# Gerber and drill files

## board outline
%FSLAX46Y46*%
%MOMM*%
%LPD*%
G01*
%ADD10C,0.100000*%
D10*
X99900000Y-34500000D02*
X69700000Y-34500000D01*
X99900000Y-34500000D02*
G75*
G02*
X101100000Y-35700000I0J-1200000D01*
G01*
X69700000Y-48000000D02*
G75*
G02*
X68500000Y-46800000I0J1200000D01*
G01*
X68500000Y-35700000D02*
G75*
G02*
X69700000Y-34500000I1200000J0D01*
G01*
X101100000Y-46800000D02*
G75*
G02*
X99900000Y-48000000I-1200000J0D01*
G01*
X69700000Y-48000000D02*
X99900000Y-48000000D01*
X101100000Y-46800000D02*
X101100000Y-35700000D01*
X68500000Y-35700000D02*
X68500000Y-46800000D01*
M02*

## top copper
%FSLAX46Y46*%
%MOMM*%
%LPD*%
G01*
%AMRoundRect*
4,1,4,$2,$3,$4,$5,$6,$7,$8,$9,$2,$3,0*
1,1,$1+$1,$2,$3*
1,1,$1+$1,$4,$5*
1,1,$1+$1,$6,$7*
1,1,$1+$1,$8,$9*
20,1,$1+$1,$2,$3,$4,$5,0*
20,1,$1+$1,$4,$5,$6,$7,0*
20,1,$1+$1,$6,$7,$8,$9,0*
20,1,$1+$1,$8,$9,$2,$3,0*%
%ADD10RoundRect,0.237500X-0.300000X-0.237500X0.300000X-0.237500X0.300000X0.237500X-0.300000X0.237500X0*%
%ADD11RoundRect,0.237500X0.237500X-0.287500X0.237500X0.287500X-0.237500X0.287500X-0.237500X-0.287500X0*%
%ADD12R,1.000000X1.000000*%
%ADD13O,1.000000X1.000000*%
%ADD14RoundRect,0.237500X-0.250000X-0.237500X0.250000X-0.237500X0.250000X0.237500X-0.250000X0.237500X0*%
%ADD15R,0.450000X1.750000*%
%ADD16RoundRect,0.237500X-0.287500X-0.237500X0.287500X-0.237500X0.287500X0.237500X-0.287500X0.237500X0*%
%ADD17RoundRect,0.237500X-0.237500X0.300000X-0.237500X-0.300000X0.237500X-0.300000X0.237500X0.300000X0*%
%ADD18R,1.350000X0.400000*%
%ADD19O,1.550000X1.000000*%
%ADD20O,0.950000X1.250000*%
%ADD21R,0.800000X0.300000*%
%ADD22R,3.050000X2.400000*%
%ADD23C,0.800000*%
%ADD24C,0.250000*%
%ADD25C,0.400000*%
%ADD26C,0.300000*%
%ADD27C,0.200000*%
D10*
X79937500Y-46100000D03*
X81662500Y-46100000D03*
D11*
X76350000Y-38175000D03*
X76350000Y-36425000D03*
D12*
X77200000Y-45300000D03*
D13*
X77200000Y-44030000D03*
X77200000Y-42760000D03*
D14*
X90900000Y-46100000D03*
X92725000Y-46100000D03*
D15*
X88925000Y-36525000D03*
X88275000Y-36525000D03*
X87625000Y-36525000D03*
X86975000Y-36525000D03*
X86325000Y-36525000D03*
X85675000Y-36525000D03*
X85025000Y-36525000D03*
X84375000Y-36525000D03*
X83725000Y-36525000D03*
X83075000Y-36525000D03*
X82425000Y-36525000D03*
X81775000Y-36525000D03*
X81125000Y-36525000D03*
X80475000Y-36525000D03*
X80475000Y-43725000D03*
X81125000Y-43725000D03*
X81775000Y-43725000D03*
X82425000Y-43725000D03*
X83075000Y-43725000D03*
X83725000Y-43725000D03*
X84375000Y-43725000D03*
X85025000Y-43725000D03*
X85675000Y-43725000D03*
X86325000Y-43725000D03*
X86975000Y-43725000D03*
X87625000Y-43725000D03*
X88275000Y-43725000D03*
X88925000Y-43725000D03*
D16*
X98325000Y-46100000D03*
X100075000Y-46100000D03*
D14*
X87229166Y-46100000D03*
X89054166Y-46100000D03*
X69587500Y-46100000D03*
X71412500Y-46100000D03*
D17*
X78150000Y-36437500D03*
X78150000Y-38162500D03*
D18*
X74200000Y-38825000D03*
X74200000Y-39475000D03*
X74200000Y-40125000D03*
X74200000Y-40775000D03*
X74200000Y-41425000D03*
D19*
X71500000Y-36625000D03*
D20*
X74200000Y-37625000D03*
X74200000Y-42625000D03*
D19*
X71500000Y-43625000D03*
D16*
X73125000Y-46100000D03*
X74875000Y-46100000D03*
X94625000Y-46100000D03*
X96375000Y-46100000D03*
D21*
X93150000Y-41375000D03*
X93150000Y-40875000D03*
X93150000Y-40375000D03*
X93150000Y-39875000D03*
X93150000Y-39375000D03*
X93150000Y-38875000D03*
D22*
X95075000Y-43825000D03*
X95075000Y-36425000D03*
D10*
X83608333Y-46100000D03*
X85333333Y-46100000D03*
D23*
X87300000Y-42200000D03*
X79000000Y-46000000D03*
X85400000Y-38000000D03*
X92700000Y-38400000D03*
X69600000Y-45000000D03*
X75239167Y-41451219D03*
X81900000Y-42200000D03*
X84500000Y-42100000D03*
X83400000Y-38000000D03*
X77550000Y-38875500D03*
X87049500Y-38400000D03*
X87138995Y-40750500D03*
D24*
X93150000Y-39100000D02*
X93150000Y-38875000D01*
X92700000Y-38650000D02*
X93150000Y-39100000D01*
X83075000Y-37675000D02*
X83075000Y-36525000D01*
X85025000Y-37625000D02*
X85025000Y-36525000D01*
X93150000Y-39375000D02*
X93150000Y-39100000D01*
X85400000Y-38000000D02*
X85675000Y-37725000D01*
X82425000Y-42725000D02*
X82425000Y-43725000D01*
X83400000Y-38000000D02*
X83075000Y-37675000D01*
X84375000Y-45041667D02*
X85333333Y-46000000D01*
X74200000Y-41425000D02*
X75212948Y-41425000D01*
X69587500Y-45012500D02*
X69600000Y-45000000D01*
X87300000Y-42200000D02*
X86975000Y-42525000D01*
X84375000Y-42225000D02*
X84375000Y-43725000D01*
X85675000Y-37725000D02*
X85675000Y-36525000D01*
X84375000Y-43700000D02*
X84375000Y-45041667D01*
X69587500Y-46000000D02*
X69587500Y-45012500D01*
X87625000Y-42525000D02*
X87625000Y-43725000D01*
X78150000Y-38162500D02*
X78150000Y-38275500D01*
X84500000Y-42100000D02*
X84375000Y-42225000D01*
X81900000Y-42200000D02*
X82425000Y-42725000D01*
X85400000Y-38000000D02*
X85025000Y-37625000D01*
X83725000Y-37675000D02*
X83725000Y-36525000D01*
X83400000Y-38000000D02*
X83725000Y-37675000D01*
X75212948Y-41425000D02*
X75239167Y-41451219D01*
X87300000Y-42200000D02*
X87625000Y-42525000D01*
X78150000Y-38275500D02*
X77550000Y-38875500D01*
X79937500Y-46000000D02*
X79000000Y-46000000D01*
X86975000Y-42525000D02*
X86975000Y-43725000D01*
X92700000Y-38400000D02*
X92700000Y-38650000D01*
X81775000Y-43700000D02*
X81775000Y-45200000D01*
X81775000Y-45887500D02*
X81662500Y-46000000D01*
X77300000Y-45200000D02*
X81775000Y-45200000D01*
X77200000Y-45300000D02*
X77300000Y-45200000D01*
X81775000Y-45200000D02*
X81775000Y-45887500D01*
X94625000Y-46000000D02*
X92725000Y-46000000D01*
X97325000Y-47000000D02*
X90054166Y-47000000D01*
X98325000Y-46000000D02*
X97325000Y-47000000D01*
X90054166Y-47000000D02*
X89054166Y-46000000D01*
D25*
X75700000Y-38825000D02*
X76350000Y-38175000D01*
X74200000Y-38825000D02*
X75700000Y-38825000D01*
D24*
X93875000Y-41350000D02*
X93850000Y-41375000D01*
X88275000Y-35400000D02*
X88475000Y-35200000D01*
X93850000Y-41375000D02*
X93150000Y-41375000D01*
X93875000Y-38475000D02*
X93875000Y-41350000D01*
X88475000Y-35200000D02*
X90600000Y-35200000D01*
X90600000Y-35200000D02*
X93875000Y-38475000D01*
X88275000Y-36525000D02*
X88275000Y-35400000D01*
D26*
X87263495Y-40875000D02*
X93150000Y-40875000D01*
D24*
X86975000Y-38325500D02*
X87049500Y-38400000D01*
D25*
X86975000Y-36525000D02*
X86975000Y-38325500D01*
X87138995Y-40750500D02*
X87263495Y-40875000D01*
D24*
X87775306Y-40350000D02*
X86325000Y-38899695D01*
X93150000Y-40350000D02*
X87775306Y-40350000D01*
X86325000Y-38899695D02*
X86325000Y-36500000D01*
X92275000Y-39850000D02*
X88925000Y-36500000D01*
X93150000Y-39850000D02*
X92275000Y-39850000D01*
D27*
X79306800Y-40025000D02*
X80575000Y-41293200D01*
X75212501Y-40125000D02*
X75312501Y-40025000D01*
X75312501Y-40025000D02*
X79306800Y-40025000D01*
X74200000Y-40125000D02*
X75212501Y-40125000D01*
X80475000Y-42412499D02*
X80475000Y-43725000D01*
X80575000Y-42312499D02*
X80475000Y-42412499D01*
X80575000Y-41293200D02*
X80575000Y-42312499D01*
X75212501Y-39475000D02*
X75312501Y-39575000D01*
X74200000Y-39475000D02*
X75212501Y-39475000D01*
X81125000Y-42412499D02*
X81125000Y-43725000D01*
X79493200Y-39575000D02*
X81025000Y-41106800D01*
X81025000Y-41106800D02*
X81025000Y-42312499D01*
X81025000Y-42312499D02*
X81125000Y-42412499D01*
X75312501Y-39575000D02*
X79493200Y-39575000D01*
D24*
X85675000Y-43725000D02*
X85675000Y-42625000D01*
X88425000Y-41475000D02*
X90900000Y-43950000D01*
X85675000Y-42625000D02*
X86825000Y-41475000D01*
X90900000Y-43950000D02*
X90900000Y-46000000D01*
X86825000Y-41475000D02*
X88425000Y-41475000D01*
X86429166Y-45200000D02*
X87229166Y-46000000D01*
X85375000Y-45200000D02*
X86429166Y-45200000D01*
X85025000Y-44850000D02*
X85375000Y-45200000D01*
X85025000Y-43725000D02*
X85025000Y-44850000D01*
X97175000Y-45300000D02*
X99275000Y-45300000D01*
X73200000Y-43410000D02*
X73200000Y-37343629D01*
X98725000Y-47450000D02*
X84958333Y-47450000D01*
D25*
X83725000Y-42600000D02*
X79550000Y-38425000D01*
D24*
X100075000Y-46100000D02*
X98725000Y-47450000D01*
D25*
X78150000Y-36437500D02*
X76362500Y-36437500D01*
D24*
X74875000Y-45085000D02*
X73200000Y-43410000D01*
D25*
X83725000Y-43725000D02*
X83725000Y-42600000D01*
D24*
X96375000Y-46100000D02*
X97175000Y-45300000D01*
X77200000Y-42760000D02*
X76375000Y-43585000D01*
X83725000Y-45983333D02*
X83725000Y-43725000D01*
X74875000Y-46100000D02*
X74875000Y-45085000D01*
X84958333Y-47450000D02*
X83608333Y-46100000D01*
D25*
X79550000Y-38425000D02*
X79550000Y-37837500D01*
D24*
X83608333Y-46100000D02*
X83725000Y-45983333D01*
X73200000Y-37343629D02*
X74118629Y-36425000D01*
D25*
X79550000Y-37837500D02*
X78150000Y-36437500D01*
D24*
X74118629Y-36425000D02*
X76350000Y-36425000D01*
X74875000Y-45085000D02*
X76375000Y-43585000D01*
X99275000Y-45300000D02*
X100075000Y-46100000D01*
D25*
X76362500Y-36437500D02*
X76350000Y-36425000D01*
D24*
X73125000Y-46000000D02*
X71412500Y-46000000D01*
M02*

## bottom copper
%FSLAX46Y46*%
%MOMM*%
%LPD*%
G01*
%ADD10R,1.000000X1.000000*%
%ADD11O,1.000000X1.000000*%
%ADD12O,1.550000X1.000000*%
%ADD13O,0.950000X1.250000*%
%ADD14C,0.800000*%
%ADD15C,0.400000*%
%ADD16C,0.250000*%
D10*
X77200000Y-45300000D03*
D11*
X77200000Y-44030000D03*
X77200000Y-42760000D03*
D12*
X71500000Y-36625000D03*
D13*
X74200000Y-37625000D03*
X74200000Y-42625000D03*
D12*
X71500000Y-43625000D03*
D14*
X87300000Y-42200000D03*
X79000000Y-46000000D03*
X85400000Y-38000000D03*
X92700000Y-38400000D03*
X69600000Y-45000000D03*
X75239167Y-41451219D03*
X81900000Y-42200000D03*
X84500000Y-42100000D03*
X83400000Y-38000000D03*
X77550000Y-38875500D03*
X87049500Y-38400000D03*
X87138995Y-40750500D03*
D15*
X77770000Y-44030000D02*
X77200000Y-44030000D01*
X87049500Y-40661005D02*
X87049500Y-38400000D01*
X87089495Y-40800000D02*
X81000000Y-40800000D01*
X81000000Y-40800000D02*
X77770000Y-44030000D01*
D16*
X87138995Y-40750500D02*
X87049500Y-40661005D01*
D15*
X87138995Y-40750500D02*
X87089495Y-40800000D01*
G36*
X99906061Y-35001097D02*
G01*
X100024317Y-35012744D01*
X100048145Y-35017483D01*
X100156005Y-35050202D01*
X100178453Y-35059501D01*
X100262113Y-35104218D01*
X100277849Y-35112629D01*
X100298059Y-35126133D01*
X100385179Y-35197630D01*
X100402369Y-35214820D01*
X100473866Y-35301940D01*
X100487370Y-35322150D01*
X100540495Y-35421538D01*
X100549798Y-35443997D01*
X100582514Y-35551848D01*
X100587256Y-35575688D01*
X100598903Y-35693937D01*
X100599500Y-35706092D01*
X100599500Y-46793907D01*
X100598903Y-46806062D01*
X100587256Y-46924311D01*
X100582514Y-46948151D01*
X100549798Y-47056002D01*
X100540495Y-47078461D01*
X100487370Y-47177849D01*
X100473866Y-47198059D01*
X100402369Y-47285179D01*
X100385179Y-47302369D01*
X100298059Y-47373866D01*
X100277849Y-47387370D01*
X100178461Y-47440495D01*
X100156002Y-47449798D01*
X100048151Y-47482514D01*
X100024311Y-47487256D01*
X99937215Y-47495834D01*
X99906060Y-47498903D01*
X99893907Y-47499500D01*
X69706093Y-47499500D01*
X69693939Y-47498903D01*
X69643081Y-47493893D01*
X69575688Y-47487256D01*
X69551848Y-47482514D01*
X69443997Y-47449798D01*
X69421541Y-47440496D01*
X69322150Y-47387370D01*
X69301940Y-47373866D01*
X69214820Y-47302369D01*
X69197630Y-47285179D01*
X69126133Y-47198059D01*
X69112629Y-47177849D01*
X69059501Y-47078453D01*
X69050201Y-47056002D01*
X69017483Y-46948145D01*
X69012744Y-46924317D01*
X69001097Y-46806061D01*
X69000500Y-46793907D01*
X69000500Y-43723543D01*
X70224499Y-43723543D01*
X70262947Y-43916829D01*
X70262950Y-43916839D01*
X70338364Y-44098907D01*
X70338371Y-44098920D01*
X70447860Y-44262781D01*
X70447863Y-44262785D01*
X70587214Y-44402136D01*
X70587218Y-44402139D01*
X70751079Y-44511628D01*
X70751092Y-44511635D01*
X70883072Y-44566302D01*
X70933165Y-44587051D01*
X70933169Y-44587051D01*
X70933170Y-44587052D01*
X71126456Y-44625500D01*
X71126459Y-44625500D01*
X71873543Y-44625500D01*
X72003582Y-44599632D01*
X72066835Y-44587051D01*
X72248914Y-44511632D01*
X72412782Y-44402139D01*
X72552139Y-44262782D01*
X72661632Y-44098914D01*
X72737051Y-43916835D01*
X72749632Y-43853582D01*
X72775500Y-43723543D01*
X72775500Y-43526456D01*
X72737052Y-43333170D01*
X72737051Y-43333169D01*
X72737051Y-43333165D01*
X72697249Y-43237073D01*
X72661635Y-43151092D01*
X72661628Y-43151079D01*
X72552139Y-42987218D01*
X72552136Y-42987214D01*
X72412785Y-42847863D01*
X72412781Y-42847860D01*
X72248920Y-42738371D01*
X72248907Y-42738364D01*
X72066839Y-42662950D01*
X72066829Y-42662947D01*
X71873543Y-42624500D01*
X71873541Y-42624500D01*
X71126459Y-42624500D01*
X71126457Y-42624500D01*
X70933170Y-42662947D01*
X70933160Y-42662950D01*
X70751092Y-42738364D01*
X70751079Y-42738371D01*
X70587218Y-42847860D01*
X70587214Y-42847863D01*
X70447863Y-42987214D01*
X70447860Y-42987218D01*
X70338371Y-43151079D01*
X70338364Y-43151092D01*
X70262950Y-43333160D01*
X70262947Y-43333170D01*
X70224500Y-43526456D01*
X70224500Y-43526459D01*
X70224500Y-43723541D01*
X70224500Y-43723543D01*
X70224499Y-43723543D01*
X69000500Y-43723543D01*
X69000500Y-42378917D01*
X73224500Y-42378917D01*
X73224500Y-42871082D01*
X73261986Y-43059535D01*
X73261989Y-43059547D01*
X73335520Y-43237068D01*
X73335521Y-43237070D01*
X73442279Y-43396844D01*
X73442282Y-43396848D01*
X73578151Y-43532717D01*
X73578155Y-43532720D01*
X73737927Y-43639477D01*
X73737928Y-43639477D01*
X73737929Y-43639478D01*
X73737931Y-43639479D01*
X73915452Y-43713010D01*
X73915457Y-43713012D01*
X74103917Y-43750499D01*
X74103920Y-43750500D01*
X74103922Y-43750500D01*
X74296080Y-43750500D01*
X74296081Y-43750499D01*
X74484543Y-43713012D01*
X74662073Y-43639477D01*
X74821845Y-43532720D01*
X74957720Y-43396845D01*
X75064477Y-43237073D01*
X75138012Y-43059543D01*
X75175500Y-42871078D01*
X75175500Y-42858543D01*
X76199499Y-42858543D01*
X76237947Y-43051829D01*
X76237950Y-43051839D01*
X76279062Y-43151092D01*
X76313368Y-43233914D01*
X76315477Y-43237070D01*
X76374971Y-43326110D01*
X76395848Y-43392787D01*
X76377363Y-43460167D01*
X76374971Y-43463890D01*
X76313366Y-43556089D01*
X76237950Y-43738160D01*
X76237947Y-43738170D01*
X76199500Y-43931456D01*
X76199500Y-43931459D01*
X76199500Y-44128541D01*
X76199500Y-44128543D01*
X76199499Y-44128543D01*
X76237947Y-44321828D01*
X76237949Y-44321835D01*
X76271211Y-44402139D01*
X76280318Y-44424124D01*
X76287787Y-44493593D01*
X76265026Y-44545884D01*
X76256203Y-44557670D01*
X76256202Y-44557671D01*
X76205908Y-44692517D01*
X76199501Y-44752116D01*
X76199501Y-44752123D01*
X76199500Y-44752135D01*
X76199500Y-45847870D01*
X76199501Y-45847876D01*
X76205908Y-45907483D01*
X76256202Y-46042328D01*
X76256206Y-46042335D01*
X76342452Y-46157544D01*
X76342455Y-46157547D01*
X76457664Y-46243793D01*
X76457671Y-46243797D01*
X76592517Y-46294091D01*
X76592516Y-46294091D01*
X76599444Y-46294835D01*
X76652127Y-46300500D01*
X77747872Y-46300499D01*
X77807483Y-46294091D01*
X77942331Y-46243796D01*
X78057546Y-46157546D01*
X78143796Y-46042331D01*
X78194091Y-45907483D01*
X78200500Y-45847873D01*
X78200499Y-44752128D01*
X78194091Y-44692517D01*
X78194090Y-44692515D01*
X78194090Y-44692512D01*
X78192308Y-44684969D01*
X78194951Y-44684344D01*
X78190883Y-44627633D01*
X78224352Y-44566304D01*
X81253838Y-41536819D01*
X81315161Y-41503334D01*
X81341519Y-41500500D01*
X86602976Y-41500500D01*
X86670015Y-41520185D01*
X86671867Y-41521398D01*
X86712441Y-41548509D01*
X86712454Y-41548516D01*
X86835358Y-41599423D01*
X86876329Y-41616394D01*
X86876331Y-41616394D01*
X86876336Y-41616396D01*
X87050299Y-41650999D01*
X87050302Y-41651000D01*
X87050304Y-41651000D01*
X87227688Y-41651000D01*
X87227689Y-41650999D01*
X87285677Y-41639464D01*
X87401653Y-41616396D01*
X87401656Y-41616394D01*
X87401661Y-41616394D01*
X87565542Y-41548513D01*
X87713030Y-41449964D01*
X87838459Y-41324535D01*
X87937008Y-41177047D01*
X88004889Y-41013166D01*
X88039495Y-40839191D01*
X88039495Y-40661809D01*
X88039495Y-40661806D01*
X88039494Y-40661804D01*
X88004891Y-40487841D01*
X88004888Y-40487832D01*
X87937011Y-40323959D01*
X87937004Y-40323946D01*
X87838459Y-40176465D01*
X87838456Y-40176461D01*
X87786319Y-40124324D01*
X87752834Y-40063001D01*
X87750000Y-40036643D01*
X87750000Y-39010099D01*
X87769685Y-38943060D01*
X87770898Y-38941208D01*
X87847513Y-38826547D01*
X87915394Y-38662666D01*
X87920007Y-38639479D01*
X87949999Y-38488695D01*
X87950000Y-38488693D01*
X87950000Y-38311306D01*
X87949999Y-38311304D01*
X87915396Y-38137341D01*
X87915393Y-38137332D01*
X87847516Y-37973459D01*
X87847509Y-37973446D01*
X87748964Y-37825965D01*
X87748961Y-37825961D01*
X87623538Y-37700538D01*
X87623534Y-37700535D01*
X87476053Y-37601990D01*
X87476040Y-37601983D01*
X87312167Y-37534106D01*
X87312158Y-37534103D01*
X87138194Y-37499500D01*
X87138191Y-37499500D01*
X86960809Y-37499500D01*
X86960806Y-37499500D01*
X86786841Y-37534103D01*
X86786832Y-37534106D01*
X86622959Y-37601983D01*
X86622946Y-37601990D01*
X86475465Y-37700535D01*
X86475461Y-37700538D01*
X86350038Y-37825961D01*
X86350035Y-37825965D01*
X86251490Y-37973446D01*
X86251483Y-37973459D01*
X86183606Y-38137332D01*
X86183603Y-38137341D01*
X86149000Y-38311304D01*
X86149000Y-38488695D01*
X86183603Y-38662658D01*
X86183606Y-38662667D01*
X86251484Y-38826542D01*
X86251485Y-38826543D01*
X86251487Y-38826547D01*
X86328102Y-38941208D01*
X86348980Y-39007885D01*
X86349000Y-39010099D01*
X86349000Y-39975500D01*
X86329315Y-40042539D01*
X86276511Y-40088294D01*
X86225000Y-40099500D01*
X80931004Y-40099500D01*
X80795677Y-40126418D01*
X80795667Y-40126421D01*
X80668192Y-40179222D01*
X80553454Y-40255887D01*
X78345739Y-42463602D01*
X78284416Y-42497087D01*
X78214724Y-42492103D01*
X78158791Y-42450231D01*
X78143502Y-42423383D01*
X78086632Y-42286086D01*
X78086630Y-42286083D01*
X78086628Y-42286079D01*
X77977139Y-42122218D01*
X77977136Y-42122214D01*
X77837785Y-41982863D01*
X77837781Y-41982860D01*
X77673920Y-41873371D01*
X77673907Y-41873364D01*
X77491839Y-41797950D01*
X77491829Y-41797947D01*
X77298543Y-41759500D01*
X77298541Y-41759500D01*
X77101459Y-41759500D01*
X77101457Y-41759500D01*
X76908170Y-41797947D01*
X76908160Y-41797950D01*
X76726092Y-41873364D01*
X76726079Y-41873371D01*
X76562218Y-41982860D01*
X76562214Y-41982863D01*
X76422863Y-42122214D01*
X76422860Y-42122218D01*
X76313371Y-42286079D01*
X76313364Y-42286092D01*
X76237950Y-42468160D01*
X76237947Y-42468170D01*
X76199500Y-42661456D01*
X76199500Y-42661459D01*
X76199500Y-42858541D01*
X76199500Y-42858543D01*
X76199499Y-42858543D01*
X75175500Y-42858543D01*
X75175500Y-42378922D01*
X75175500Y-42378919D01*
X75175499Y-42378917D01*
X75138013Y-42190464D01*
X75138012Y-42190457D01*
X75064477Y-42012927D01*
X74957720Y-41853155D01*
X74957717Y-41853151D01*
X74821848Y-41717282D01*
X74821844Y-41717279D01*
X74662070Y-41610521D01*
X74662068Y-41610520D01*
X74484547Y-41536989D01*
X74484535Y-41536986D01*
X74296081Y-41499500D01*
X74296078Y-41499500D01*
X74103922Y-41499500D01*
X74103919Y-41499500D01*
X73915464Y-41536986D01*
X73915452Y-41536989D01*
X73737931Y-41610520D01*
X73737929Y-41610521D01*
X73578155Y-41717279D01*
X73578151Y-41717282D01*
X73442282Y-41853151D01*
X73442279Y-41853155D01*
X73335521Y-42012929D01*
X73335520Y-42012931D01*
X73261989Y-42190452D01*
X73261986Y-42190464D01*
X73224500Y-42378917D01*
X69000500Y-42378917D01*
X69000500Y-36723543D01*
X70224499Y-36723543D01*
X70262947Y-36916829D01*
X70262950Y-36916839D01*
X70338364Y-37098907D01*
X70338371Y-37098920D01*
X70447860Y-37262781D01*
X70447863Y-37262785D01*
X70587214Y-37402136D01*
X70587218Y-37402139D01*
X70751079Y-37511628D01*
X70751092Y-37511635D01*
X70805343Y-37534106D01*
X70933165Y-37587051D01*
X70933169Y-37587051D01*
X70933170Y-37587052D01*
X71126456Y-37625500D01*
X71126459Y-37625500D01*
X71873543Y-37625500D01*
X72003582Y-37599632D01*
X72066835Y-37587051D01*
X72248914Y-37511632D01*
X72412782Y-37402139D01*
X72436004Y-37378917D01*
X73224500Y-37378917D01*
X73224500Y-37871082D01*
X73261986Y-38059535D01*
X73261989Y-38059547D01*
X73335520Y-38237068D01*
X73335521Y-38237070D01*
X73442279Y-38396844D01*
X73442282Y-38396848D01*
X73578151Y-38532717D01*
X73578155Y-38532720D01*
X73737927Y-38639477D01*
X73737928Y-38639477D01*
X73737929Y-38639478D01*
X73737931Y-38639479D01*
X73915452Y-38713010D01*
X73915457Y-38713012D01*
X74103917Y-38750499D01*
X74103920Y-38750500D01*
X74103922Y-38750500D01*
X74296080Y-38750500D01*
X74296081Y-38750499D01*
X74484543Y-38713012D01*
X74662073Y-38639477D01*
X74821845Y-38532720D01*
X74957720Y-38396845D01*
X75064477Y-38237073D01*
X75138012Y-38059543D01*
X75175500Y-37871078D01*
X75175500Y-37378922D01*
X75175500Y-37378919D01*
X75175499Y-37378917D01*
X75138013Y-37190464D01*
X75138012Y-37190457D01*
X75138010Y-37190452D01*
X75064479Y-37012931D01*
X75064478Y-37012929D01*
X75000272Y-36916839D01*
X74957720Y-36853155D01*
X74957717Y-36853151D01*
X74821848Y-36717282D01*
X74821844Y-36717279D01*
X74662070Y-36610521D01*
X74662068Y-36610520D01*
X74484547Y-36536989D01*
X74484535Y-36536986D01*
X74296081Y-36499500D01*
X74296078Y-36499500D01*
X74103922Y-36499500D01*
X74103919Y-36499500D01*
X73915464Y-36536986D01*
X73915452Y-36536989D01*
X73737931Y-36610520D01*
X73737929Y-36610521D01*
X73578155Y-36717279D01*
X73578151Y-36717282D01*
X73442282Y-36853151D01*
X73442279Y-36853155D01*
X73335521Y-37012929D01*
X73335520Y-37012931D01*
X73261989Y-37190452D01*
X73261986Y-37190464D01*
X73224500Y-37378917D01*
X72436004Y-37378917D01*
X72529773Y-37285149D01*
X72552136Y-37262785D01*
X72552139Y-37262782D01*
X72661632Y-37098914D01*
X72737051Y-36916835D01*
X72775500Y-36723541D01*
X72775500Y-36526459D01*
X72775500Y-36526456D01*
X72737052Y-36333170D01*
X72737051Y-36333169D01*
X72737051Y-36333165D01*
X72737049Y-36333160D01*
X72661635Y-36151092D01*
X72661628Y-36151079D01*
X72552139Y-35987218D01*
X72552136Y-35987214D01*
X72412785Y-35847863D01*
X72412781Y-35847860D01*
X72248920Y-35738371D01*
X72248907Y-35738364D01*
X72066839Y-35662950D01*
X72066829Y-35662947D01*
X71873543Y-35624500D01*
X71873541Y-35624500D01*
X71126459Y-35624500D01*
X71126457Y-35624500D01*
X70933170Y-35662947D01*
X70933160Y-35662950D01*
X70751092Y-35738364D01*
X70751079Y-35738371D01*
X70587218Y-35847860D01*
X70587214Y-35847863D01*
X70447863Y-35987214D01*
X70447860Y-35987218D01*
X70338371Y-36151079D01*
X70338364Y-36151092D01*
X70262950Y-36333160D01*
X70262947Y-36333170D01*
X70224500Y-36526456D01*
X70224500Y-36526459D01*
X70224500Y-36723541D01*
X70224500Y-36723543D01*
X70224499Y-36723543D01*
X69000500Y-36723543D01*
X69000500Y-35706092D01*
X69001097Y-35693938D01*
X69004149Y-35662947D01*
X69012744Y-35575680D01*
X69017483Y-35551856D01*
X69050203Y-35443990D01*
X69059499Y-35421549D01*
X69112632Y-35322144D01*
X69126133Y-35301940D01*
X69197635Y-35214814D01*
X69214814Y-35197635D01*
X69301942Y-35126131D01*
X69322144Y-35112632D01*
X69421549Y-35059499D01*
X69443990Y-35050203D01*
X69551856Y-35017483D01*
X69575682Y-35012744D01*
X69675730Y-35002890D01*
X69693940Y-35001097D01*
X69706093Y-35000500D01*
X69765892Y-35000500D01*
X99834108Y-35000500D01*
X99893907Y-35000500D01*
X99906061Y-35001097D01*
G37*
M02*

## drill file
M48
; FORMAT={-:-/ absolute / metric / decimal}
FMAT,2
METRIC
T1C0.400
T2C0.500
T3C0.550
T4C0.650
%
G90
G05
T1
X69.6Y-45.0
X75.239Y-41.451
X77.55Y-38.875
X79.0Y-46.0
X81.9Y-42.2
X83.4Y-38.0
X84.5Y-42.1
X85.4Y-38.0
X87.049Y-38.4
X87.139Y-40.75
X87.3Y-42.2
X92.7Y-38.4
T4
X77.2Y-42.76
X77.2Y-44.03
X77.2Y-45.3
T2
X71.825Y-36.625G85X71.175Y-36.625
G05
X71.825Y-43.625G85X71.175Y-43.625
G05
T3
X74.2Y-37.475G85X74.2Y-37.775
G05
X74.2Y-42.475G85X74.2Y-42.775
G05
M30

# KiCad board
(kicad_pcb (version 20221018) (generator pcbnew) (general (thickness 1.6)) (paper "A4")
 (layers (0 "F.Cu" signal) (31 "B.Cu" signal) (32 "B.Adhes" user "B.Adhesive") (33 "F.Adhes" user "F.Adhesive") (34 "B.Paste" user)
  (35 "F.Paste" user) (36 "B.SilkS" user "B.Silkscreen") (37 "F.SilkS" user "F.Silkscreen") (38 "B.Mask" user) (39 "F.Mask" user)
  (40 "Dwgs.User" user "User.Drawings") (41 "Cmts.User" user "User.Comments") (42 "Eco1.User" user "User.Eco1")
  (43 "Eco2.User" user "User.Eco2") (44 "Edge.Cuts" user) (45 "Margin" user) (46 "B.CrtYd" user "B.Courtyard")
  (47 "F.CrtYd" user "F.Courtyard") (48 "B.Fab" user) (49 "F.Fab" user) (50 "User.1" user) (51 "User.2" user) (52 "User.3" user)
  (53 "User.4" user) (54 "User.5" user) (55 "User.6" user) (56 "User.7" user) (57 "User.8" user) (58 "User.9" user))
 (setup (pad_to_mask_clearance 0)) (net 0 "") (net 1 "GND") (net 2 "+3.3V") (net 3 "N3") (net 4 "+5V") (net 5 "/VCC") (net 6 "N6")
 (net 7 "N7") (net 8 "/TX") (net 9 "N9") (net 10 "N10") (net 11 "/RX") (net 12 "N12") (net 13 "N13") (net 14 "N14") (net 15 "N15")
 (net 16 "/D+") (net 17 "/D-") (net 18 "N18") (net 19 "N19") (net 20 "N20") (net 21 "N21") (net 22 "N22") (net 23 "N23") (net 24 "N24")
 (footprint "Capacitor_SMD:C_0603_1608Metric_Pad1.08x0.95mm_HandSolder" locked (layer "F.Cu") (at 80.8 46.1)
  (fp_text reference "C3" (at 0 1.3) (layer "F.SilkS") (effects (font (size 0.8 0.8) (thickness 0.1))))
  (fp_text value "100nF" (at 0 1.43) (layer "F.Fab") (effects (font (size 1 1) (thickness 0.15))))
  (pad "1" smd roundrect locked (at -0.8625 0) (size 1.075 0.95) (layers "F.Cu" "F.Paste" "F.Mask") (roundrect_rratio 0.25) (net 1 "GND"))
  (pad "2" smd roundrect locked (at 0.8625 0) (size 1.075 0.95) (layers "F.Cu" "F.Paste" "F.Mask") (roundrect_rratio 0.25) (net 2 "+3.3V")))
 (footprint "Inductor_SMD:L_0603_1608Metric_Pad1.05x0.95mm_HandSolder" (layer "F.Cu") (at 76.35 37.3 90)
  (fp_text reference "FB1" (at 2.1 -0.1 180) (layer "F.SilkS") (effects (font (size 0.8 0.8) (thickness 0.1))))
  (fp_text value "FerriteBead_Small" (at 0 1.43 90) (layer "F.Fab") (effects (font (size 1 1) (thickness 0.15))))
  (pad "1" smd roundrect (at -0.875 0 90) (size 1.05 0.95) (layers "F.Cu" "F.Paste" "F.Mask") (roundrect_rratio 0.25) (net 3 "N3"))
  (pad "2" smd roundrect (at 0.875 0 90) (size 1.05 0.95) (layers "F.Cu" "F.Paste" "F.Mask") (roundrect_rratio 0.25) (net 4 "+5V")))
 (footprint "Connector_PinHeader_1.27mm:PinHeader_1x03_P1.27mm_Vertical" (layer "F.Cu") (at 77.2 45.3 180)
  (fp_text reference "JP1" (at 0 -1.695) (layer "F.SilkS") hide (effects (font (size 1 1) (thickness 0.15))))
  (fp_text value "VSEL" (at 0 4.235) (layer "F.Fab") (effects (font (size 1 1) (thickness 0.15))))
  (pad "1" thru_hole rect (at 0 0 180) (size 1 1) (drill 0.65) (layers "*.Cu" "*.Mask") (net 2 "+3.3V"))
  (pad "2" thru_hole oval (at 0 1.27 180) (size 1 1) (drill 0.65) (layers "*.Cu" "*.Mask") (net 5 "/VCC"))
  (pad "3" thru_hole oval (at 0 2.54 180) (size 1 1) (drill 0.65) (layers "*.Cu" "*.Mask") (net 4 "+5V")))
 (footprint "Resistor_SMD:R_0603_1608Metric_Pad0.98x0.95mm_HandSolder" (layer "F.Cu") (at 91.8125 46.1)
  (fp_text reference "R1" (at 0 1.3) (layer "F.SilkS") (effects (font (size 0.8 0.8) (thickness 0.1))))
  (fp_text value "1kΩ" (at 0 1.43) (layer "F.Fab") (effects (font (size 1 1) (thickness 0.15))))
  (pad "1" smd roundrect (at -0.9125 0) (size 0.975 0.95) (layers "F.Cu" "F.Paste" "F.Mask") (roundrect_rratio 0.25) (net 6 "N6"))
  (pad "2" smd roundrect (at 0.9125 0) (size 0.975 0.95) (layers "F.Cu" "F.Paste" "F.Mask") (roundrect_rratio 0.25) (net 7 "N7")))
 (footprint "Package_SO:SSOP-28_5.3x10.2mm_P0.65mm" (layer "F.Cu") (at 84.7 40.125 -90)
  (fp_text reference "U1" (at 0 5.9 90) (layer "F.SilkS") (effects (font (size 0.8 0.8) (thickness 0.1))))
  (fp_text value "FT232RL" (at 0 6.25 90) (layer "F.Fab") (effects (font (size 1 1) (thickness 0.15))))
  (pad "1" smd rect (at -3.6 -4.225 270) (size 1.75 0.45) (layers "F.Cu" "F.Paste" "F.Mask") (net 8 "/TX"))
  (pad "2" smd rect (at -3.6 -3.575 270) (size 1.75 0.45) (layers "F.Cu" "F.Paste" "F.Mask") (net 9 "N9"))
  (pad "3" smd rect (at -3.6 -2.925 270) (size 1.75 0.45) (layers "F.Cu" "F.Paste" "F.Mask") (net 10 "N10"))
  (pad "4" smd rect (at -3.6 -2.275 270) (size 1.75 0.45) (layers "F.Cu" "F.Paste" "F.Mask") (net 5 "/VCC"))
  (pad "5" smd rect (at -3.6 -1.625 270) (size 1.75 0.45) (layers "F.Cu" "F.Paste" "F.Mask") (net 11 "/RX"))
  (pad "6" smd rect (at -3.6 -0.975 270) (size 1.75 0.45) (layers "F.Cu" "F.Paste" "F.Mask") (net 1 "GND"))
  (pad "7" smd rect (at -3.6 -0.325 270) (size 1.75 0.45) (layers "F.Cu" "F.Paste" "F.Mask") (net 1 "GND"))
  (pad "8" smd rect (at -3.6 0.325 270) (size 1.75 0.45) (layers "F.Cu" "F.Paste" "F.Mask"))
  (pad "9" smd rect (at -3.6 0.975 270) (size 1.75 0.45) (layers "F.Cu" "F.Paste" "F.Mask") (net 1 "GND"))
  (pad "10" smd rect (at -3.6 1.625 270) (size 1.75 0.45) (layers "F.Cu" "F.Paste" "F.Mask") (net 1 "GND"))
  (pad "11" smd rect (at -3.6 2.275 270) (size 1.75 0.45) (layers "F.Cu" "F.Paste" "F.Mask") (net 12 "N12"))
  (pad "12" smd rect (at -3.6 2.925 270) (size 1.75 0.45) (layers "F.Cu" "F.Paste" "F.Mask") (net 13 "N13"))
  (pad "13" smd rect (at -3.6 3.575 270) (size 1.75 0.45) (layers "F.Cu" "F.Paste" "F.Mask") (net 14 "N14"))
  (pad "14" smd rect (at -3.6 4.225 270) (size 1.75 0.45) (layers "F.Cu" "F.Paste" "F.Mask") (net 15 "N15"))
  (pad "15" smd rect (at 3.6 4.225 270) (size 1.75 0.45) (layers "F.Cu" "F.Paste" "F.Mask") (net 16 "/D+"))
  (pad "16" smd rect (at 3.6 3.575 270) (size 1.75 0.45) (layers "F.Cu" "F.Paste" "F.Mask") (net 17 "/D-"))
  (pad "17" smd rect (at 3.6 2.925 270) (size 1.75 0.45) (layers "F.Cu" "F.Paste" "F.Mask") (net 2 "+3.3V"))
  (pad "18" smd rect (at 3.6 2.275 270) (size 1.75 0.45) (layers "F.Cu" "F.Paste" "F.Mask") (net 1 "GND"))
  (pad "19" smd rect (at 3.6 1.625 270) (size 1.75 0.45) (layers "F.Cu" "F.Paste" "F.Mask") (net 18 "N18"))
  (pad "20" smd rect (at 3.6 0.975 270) (size 1.75 0.45) (layers "F.Cu" "F.Paste" "F.Mask") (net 4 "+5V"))
  (pad "21" smd rect (at 3.6 0.325 270) (size 1.75 0.45) (layers "F.Cu" "F.Paste" "F.Mask") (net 1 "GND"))
  (pad "22" smd rect (at 3.6 -0.325 270) (size 1.75 0.45) (layers "F.Cu" "F.Paste" "F.Mask") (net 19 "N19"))
  (pad "23" smd rect (at 3.6 -0.975 270) (size 1.75 0.45) (layers "F.Cu" "F.Paste" "F.Mask") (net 6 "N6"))
  (pad "24" smd rect (at 3.6 -1.625 270) (size 1.75 0.45) (layers "F.Cu" "F.Paste" "F.Mask"))
  (pad "25" smd rect (at 3.6 -2.275 270) (size 1.75 0.45) (layers "F.Cu" "F.Paste" "F.Mask") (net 1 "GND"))
  (pad "26" smd rect (at 3.6 -2.925 270) (size 1.75 0.45) (layers "F.Cu" "F.Paste" "F.Mask") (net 1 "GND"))
  (pad "27" smd rect (at 3.6 -3.575 270) (size 1.75 0.45) (layers "F.Cu" "F.Paste" "F.Mask") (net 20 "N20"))
  (pad "28" smd rect (at 3.6 -4.225 270) (size 1.75 0.45) (layers "F.Cu" "F.Paste" "F.Mask") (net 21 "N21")))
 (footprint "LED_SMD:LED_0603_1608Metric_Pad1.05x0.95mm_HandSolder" (layer "F.Cu") (at 99.2 46.1)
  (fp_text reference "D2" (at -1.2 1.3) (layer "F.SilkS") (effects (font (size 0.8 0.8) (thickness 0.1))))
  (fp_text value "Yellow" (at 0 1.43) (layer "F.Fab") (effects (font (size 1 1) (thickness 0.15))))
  (pad "1" smd roundrect (at -0.875 0) (size 1.05 0.95) (layers "F.Cu" "F.Paste" "F.Mask") (roundrect_rratio 0.25) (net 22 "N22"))
  (pad "2" smd roundrect (at 0.875 0) (size 1.05 0.95) (layers "F.Cu" "F.Paste" "F.Mask") (roundrect_rratio 0.25) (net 4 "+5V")))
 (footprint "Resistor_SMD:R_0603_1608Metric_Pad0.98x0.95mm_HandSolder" (layer "F.Cu") (at 88.141666 46.1)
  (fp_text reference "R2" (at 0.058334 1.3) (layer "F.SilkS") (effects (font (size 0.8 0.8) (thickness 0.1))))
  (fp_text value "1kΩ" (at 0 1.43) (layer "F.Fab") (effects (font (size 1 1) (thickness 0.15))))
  (pad "1" smd roundrect (at -0.9125 0) (size 0.975 0.95) (layers "F.Cu" "F.Paste" "F.Mask") (roundrect_rratio 0.25) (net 19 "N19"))
  (pad "2" smd roundrect (at 0.9125 0) (size 0.975 0.95) (layers "F.Cu" "F.Paste" "F.Mask") (roundrect_rratio 0.25) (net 22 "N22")))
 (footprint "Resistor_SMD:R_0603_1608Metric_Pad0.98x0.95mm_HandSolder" (layer "F.Cu") (at 70.5 46.1)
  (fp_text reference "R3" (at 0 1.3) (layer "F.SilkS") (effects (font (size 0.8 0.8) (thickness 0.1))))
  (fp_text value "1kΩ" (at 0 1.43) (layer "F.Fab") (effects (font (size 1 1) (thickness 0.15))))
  (pad "1" smd roundrect (at -0.9125 0) (size 0.975 0.95) (layers "F.Cu" "F.Paste" "F.Mask") (roundrect_rratio 0.25) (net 1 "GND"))
  (pad "2" smd roundrect (at 0.9125 0) (size 0.975 0.95) (layers "F.Cu" "F.Paste" "F.Mask") (roundrect_rratio 0.25) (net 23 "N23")))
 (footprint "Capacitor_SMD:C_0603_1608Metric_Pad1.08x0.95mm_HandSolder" (layer "F.Cu") (at 78.15 37.3 -90)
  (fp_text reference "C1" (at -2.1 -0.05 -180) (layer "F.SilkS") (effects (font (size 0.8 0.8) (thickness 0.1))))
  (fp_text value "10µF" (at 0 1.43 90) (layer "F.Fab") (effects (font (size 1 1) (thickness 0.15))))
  (pad "1" smd roundrect (at -0.8625 0 270) (size 1.075 0.95) (layers "F.Cu" "F.Paste" "F.Mask") (roundrect_rratio 0.25) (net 4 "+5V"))
  (pad "2" smd roundrect (at 0.8625 0 270) (size 1.075 0.95) (layers "F.Cu" "F.Paste" "F.Mask") (roundrect_rratio 0.25) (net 1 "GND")))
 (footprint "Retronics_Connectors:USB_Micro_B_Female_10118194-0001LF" (layer "F.Cu") (at 74.2 40.125 -90)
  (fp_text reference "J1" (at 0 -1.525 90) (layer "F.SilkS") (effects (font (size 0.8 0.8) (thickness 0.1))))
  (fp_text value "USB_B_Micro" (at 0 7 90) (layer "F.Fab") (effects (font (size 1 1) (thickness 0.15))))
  (pad "1" smd rect (at -1.3 0 270) (size 0.4 1.35) (layers "F.Cu" "F.Paste" "F.Mask") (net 3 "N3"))
  (pad "2" smd rect (at -0.65 0 270) (size 0.4 1.35) (layers "F.Cu" "F.Paste" "F.Mask") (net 17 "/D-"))
  (pad "3" smd rect (at 0 0 270) (size 0.4 1.35) (layers "F.Cu" "F.Paste" "F.Mask") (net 16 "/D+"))
  (pad "4" smd rect (at 0.65 0 270) (size 0.4 1.35) (layers "F.Cu" "F.Paste" "F.Mask") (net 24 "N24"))
  (pad "5" smd rect (at 1.3 0 270) (size 0.4 1.35) (layers "F.Cu" "F.Paste" "F.Mask") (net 1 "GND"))
  (pad "SH" thru_hole oval (at -3.5 2.7 270) (size 1 1.55) (drill oval 0.5 1.15) (layers "*.Cu" "*.Mask"))
  (pad "SH" thru_hole oval (at -2.5 0 270) (size 1.25 0.95) (drill oval 0.85 0.55) (layers "*.Cu" "*.Mask"))
  (pad "SH" thru_hole oval (at 2.5 0 270) (size 1.25 0.95) (drill oval 0.85 0.55) (layers "*.Cu" "*.Mask"))
  (pad "SH" thru_hole oval (at 3.5 2.7 270) (size 1 1.55) (drill oval 0.5 1.15) (layers "*.Cu" "*.Mask")))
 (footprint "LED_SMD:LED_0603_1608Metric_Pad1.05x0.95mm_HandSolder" (layer "F.Cu") (at 74 46.1)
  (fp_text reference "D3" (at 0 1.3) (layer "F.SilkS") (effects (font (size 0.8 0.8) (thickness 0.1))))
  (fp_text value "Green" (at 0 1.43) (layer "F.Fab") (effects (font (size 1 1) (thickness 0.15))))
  (pad "1" smd roundrect (at -0.875 0) (size 1.05 0.95) (layers "F.Cu" "F.Paste" "F.Mask") (roundrect_rratio 0.25) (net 23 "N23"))
  (pad "2" smd roundrect (at 0.875 0) (size 1.05 0.95) (layers "F.Cu" "F.Paste" "F.Mask") (roundrect_rratio 0.25) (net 4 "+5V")))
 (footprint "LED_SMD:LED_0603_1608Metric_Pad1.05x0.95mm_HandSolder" (layer "F.Cu") (at 95.5 46.1)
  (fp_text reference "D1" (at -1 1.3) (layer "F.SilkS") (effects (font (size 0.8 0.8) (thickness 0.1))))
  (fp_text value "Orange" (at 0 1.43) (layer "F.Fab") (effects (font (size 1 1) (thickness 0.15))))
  (pad "1" smd roundrect (at -0.875 0) (size 1.05 0.95) (layers "F.Cu" "F.Paste" "F.Mask") (roundrect_rratio 0.25) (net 7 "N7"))
  (pad "2" smd roundrect (at 0.875 0) (size 1.05 0.95) (layers "F.Cu" "F.Paste" "F.Mask") (roundrect_rratio 0.25) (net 4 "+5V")))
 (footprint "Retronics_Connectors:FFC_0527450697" (layer "F.Cu") (at 96.1 40.125 90)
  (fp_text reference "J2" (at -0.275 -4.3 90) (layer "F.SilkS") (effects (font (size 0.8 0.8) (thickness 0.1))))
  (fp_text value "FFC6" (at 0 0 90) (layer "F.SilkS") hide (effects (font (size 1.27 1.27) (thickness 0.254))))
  (pad "1" smd rect (at -1.25 -2.95 90) (size 0.3 0.8) (layers "F.Cu" "F.Paste" "F.Mask") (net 9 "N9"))
  (pad "2" smd rect (at -0.75 -2.95 90) (size 0.3 0.8) (layers "F.Cu" "F.Paste" "F.Mask") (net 5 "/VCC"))
  (pad "3" smd rect (at -0.25 -2.95 90) (size 0.3 0.8) (layers "F.Cu" "F.Paste" "F.Mask") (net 11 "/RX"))
  (pad "4" smd rect (at 0.25 -2.95 90) (size 0.3 0.8) (layers "F.Cu" "F.Paste" "F.Mask") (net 8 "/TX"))
  (pad "5" smd rect (at 0.75 -2.95 90) (size 0.3 0.8) (layers "F.Cu" "F.Paste" "F.Mask") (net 1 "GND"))
  (pad "6" smd rect (at 1.25 -2.95 90) (size 0.3 0.8) (layers "F.Cu" "F.Paste" "F.Mask") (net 1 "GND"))
  (pad "7" smd rect (at -3.7 -1.025 90) (size 2.4 3.05) (layers "F.Cu" "F.Paste" "F.Mask"))
  (pad "8" smd rect (at 3.7 -1.025 90) (size 2.4 3.05) (layers "F.Cu" "F.Paste" "F.Mask")))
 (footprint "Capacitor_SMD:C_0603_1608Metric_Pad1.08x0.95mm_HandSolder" (layer "F.Cu") (at 84.470833 46.1)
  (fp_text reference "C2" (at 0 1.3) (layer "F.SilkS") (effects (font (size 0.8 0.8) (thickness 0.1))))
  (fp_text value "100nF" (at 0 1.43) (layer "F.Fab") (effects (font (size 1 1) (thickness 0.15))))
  (pad "1" smd roundrect (at -0.8625 0) (size 1.075 0.95) (layers "F.Cu" "F.Paste" "F.Mask") (roundrect_rratio 0.25) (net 4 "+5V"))
  (pad "2" smd roundrect (at 0.8625 0) (size 1.075 0.95) (layers "F.Cu" "F.Paste" "F.Mask") (roundrect_rratio 0.25) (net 1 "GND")))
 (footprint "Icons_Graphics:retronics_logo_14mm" (layer "B.Cu") (at 93.996672 35.9 180)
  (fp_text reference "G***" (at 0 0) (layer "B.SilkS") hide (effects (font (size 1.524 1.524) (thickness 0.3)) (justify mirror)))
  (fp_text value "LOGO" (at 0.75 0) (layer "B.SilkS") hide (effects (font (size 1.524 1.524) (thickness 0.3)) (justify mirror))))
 (gr_line (start 99.9 34.5) (end 69.7 34.5) (stroke (width 0.1) (type default)) (layer "Edge.Cuts"))
 (gr_arc (start 99.9 34.5) (mid 100.748528 34.851472) (end 101.1 35.7) (stroke (width 0.1) (type default)) (layer "Edge.Cuts"))
 (gr_arc (start 69.7 48) (mid 68.851472 47.648528) (end 68.5 46.8) (stroke (width 0.1) (type default)) (layer "Edge.Cuts"))
 (gr_arc (start 68.5 35.7) (mid 68.851472 34.851472) (end 69.7 34.5) (stroke (width 0.1) (type default)) (layer "Edge.Cuts"))
 (gr_arc (start 101.1 46.8) (mid 100.748528 47.648528) (end 99.9 48) (stroke (width 0.1) (type default)) (layer "Edge.Cuts"))
 (gr_line (start 69.7 48) (end 99.9 48) (stroke (width 0.1) (type default)) (layer "Edge.Cuts"))
 (gr_line (start 101.1 46.8) (end 101.1 35.7) (stroke (width 0.1) (type default)) (layer "Edge.Cuts"))
 (gr_line (start 68.5 35.7) (end 68.5 46.8) (stroke (width 0.1) (type default)) (layer "Edge.Cuts"))
 (segment (start 93.15 39.1) (end 93.15 38.875) (width 0.25) (layer "F.Cu") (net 1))
 (segment (start 92.7 38.65) (end 93.15 39.1) (width 0.25) (layer "F.Cu") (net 1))
 (segment (start 83.075 37.675) (end 83.075 36.525) (width 0.25) (layer "F.Cu") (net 1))
 (segment (start 85.025 37.625) (end 85.025 36.525) (width 0.25) (layer "F.Cu") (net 1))
 (segment (start 93.15 39.375) (end 93.15 39.1) (width 0.25) (layer "F.Cu") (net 1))
 (segment (start 85.4 38) (end 85.675 37.725) (width 0.25) (layer "F.Cu") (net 1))
 (segment (start 82.425 42.725) (end 82.425 43.725) (width 0.25) (layer "F.Cu") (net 1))
 (segment (start 83.4 38) (end 83.075 37.675) (width 0.25) (layer "F.Cu") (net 1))
 (segment (start 84.375 45.041667) (end 85.333333 46) (width 0.25) (layer "F.Cu") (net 1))
 (segment (start 74.2 41.425) (end 75.212948 41.425) (width 0.25) (layer "F.Cu") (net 1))
 (segment (start 69.5875 45.0125) (end 69.6 45) (width 0.25) (layer "F.Cu") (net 1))
 (segment (start 87.3 42.2) (end 86.975 42.525) (width 0.25) (layer "F.Cu") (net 1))
 (segment (start 84.375 42.225) (end 84.375 43.725) (width 0.25) (layer "F.Cu") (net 1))
 (segment (start 85.675 37.725) (end 85.675 36.525) (width 0.25) (layer "F.Cu") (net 1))
 (segment (start 84.375 43.7) (end 84.375 45.041667) (width 0.25) (layer "F.Cu") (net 1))
 (segment (start 69.5875 46) (end 69.5875 45.0125) (width 0.25) (layer "F.Cu") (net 1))
 (segment (start 87.625 42.525) (end 87.625 43.725) (width 0.25) (layer "F.Cu") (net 1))
 (segment (start 78.15 38.1625) (end 78.15 38.2755) (width 0.25) (layer "F.Cu") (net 1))
 (segment (start 84.5 42.1) (end 84.375 42.225) (width 0.25) (layer "F.Cu") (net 1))
 (segment (start 81.9 42.2) (end 82.425 42.725) (width 0.25) (layer "F.Cu") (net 1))
 (segment (start 85.4 38) (end 85.025 37.625) (width 0.25) (layer "F.Cu") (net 1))
 (segment (start 83.725 37.675) (end 83.725 36.525) (width 0.25) (layer "F.Cu") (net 1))
 (segment (start 83.4 38) (end 83.725 37.675) (width 0.25) (layer "F.Cu") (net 1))
 (segment (start 75.212948 41.425) (end 75.239167 41.451219) (width 0.25) (layer "F.Cu") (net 1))
 (segment (start 87.3 42.2) (end 87.625 42.525) (width 0.25) (layer "F.Cu") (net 1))
 (segment (start 78.15 38.2755) (end 77.55 38.8755) (width 0.25) (layer "F.Cu") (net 1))
 (segment (start 79.9375 46) (end 79 46) (width 0.25) (layer "F.Cu") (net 1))
 (segment (start 86.975 42.525) (end 86.975 43.725) (width 0.25) (layer "F.Cu") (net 1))
 (segment (start 92.7 38.4) (end 92.7 38.65) (width 0.25) (layer "F.Cu") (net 1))
 (via (at 87.3 42.2) (size 0.8) (drill 0.4) (layers "F.Cu" "B.Cu") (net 1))
 (via (at 79 46) (size 0.8) (drill 0.4) (layers "F.Cu" "B.Cu") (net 1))
 (via (at 85.4 38) (size 0.8) (drill 0.4) (layers "F.Cu" "B.Cu") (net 1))
 (via (at 92.7 38.4) (size 0.8) (drill 0.4) (layers "F.Cu" "B.Cu") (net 1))
 (via (at 69.6 45) (size 0.8) (drill 0.4) (layers "F.Cu" "B.Cu") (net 1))
 (via (at 75.239167 41.451219) (size 0.8) (drill 0.4) (layers "F.Cu" "B.Cu") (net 1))
 (via (at 81.9 42.2) (size 0.8) (drill 0.4) (layers "F.Cu" "B.Cu") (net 1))
 (via (at 84.5 42.1) (size 0.8) (drill 0.4) (layers "F.Cu" "B.Cu") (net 1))
 (via (at 83.4 38) (size 0.8) (drill 0.4) (layers "F.Cu" "B.Cu") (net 1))
 (via (at 77.55 38.8755) (size 0.8) (drill 0.4) (layers "F.Cu" "B.Cu") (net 1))
 (segment (start 81.775 43.7) (end 81.775 45.2) (width 0.25) (layer "F.Cu") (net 2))
 (segment (start 81.775 45.8875) (end 81.6625 46) (width 0.25) (layer "F.Cu") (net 2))
 (segment (start 77.3 45.2) (end 81.775 45.2) (width 0.25) (layer "F.Cu") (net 2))
 (segment (start 77.2 45.3) (end 77.3 45.2) (width 0.25) (layer "F.Cu") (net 2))
 (segment (start 81.775 45.2) (end 81.775 45.8875) (width 0.25) (layer "F.Cu") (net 2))
 (segment (start 94.625 46) (end 92.725 46) (width 0.25) (layer "F.Cu") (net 7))
 (segment (start 97.325 47) (end 90.054166 47) (width 0.25) (layer "F.Cu") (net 22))
 (segment (start 98.325 46) (end 97.325 47) (width 0.25) (layer "F.Cu") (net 22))
 (segment (start 90.054166 47) (end 89.054166 46) (width 0.25) (layer "F.Cu") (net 22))
 (segment (start 75.7 38.825) (end 76.35 38.175) (width 0.4) (layer "F.Cu") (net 3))
 (segment (start 74.2 38.825) (end 75.7 38.825) (width 0.4) (layer "F.Cu") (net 3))
 (segment (start 93.875 41.35) (end 93.85 41.375) (width 0.25) (layer "F.Cu") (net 9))
 (segment (start 88.275 35.4) (end 88.475 35.2) (width 0.25) (layer "F.Cu") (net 9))
 (segment (start 93.85 41.375) (end 93.15 41.375) (width 0.25) (layer "F.Cu") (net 9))
 (segment (start 93.875 38.475) (end 93.875 41.35) (width 0.25) (layer "F.Cu") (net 9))
 (segment (start 88.475 35.2) (end 90.6 35.2) (width 0.25) (layer "F.Cu") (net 9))
 (segment (start 90.6 35.2) (end 93.875 38.475) (width 0.25) (layer "F.Cu") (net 9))
 (segment (start 88.275 36.525) (end 88.275 35.4) (width 0.25) (layer "F.Cu") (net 9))
 (segment (start 87.263495 40.875) (end 93.15 40.875) (width 0.3) (layer "F.Cu") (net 5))
 (segment (start 86.975 38.3255) (end 87.0495 38.4) (width 0.25) (layer "F.Cu") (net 5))
 (segment (start 86.975 36.525) (end 86.975 38.3255) (width 0.4) (layer "F.Cu") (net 5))
 (segment (start 87.138995 40.7505) (end 87.263495 40.875) (width 0.4) (layer "F.Cu") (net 5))
 (via (at 87.0495 38.4) (size 0.8) (drill 0.4) (layers "F.Cu" "B.Cu") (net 5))
 (via (at 87.138995 40.7505) (size 0.8) (drill 0.4) (layers "F.Cu" "B.Cu") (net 5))
 (segment (start 77.77 44.03) (end 77.2 44.03) (width 0.4) (layer "B.Cu") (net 5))
 (segment (start 87.0495 40.661005) (end 87.0495 38.4) (width 0.4) (layer "B.Cu") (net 5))
 (segment (start 87.089495 40.8) (end 81 40.8) (width 0.4) (layer "B.Cu") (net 5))
 (segment (start 81 40.8) (end 77.77 44.03) (width 0.4) (layer "B.Cu") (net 5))
 (segment (start 87.138995 40.7505) (end 87.0495 40.661005) (width 0.25) (layer "B.Cu") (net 5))
 (segment (start 87.138995 40.7505) (end 87.089495 40.8) (width 0.4) (layer "B.Cu") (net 5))
 (segment (start 87.775306 40.35) (end 86.325 38.899695) (width 0.25) (layer "F.Cu") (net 11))
 (segment (start 93.15 40.35) (end 87.775306 40.35) (width 0.25) (layer "F.Cu") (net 11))
 (segment (start 86.325 38.899695) (end 86.325 36.5) (width 0.25) (layer "F.Cu") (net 11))
 (segment (start 92.275 39.85) (end 88.925 36.5) (width 0.25) (layer "F.Cu") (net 8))
 (segment (start 93.15 39.85) (end 92.275 39.85) (width 0.25) (layer "F.Cu") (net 8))
 (segment (start 79.3068 40.025) (end 80.575 41.2932) (width 0.2) (layer "F.Cu") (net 16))
 (segment (start 75.212501 40.125) (end 75.312501 40.025) (width 0.2) (layer "F.Cu") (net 16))
 (segment (start 75.312501 40.025) (end 79.3068 40.025) (width 0.2) (layer "F.Cu") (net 16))
 (segment (start 74.2 40.125) (end 75.212501 40.125) (width 0.2) (layer "F.Cu") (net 16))
 (segment (start 80.475 42.412499) (end 80.475 43.725) (width 0.2) (layer "F.Cu") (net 16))
 (segment (start 80.575 42.312499) (end 80.475 42.412499) (width 0.2) (layer "F.Cu") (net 16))
 (segment (start 80.575 41.2932) (end 80.575 42.312499) (width 0.2) (layer "F.Cu") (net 16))
 (segment (start 75.212501 39.475) (end 75.312501 39.575) (width 0.2) (layer "F.Cu") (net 17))
 (segment (start 74.2 39.475) (end 75.212501 39.475) (width 0.2) (layer "F.Cu") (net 17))
 (segment (start 81.125 42.412499) (end 81.125 43.725) (width 0.2) (layer "F.Cu") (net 17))
 (segment (start 79.4932 39.575) (end 81.025 41.1068) (width 0.2) (layer "F.Cu") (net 17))
 (segment (start 81.025 41.1068) (end 81.025 42.312499) (width 0.2) (layer "F.Cu") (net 17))
 (segment (start 81.025 42.312499) (end 81.125 42.412499) (width 0.2) (layer "F.Cu") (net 17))
 (segment (start 75.312501 39.575) (end 79.4932 39.575) (width 0.2) (layer "F.Cu") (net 17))
 (segment (start 85.675 43.725) (end 85.675 42.625) (width 0.25) (layer "F.Cu") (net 6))
 (segment (start 88.425 41.475) (end 90.9 43.95) (width 0.25) (layer "F.Cu") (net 6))
 (segment (start 85.675 42.625) (end 86.825 41.475) (width 0.25) (layer "F.Cu") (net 6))
 (segment (start 90.9 43.95) (end 90.9 46) (width 0.25) (layer "F.Cu") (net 6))
 (segment (start 86.825 41.475) (end 88.425 41.475) (width 0.25) (layer "F.Cu") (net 6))
 (segment (start 86.429166 45.2) (end 87.229166 46) (width 0.25) (layer "F.Cu") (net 19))
 (segment (start 85.375 45.2) (end 86.429166 45.2) (width 0.25) (layer "F.Cu") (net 19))
 (segment (start 85.025 44.85) (end 85.375 45.2) (width 0.25) (layer "F.Cu") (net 19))
 (segment (start 85.025 43.725) (end 85.025 44.85) (width 0.25) (layer "F.Cu") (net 19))
 (segment (start 97.175 45.3) (end 99.275 45.3) (width 0.25) (layer "F.Cu") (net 4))
 (segment (start 73.2 43.41) (end 73.2 37.343629) (width 0.25) (layer "F.Cu") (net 4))
 (segment (start 98.725 47.45) (end 84.958333 47.45) (width 0.25) (layer "F.Cu") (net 4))
 (segment (start 83.725 42.6) (end 79.55 38.425) (width 0.4) (layer "F.Cu") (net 4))
 (segment (start 100.075 46.1) (end 98.725 47.45) (width 0.25) (layer "F.Cu") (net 4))
 (segment (start 78.15 36.4375) (end 76.3625 36.4375) (width 0.4) (layer "F.Cu") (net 4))
 (segment (start 74.875 45.085) (end 73.2 43.41) (width 0.25) (layer "F.Cu") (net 4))
 (segment (start 83.725 43.725) (end 83.725 42.6) (width 0.4) (layer "F.Cu") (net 4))
 (segment (start 96.375 46.1) (end 97.175 45.3) (width 0.25) (layer "F.Cu") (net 4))
 (segment (start 77.2 42.76) (end 76.375 43.585) (width 0.25) (layer "F.Cu") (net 4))
 (segment (start 83.725 45.983333) (end 83.725 43.725) (width 0.25) (layer "F.Cu") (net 4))
 (segment (start 74.875 46.1) (end 74.875 45.085) (width 0.25) (layer "F.Cu") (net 4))
 (segment (start 84.958333 47.45) (end 83.608333 46.1) (width 0.25) (layer "F.Cu") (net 4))
 (segment (start 79.55 38.425) (end 79.55 37.8375) (width 0.4) (layer "F.Cu") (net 4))
 (segment (start 83.608333 46.1) (end 83.725 45.983333) (width 0.25) (layer "F.Cu") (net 4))
 (segment (start 73.2 37.343629) (end 74.118629 36.425) (width 0.25) (layer "F.Cu") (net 4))
 (segment (start 79.55 37.8375) (end 78.15 36.4375) (width 0.4) (layer "F.Cu") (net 4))
 (segment (start 74.118629 36.425) (end 76.35 36.425) (width 0.25) (layer "F.Cu") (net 4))
 (segment (start 74.875 45.085) (end 76.375 43.585) (width 0.25) (layer "F.Cu") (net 4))
 (segment (start 99.275 45.3) (end 100.075 46.1) (width 0.25) (layer "F.Cu") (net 4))
 (segment (start 76.3625 36.4375) (end 76.35 36.425) (width 0.4) (layer "F.Cu") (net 4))
 (segment (start 73.125 46) (end 71.4125 46) (width 0.25) (layer "F.Cu") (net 23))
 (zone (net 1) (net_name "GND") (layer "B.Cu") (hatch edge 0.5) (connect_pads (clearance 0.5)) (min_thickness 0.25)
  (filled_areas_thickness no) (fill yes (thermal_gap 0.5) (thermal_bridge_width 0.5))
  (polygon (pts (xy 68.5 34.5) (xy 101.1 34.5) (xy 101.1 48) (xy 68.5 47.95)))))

